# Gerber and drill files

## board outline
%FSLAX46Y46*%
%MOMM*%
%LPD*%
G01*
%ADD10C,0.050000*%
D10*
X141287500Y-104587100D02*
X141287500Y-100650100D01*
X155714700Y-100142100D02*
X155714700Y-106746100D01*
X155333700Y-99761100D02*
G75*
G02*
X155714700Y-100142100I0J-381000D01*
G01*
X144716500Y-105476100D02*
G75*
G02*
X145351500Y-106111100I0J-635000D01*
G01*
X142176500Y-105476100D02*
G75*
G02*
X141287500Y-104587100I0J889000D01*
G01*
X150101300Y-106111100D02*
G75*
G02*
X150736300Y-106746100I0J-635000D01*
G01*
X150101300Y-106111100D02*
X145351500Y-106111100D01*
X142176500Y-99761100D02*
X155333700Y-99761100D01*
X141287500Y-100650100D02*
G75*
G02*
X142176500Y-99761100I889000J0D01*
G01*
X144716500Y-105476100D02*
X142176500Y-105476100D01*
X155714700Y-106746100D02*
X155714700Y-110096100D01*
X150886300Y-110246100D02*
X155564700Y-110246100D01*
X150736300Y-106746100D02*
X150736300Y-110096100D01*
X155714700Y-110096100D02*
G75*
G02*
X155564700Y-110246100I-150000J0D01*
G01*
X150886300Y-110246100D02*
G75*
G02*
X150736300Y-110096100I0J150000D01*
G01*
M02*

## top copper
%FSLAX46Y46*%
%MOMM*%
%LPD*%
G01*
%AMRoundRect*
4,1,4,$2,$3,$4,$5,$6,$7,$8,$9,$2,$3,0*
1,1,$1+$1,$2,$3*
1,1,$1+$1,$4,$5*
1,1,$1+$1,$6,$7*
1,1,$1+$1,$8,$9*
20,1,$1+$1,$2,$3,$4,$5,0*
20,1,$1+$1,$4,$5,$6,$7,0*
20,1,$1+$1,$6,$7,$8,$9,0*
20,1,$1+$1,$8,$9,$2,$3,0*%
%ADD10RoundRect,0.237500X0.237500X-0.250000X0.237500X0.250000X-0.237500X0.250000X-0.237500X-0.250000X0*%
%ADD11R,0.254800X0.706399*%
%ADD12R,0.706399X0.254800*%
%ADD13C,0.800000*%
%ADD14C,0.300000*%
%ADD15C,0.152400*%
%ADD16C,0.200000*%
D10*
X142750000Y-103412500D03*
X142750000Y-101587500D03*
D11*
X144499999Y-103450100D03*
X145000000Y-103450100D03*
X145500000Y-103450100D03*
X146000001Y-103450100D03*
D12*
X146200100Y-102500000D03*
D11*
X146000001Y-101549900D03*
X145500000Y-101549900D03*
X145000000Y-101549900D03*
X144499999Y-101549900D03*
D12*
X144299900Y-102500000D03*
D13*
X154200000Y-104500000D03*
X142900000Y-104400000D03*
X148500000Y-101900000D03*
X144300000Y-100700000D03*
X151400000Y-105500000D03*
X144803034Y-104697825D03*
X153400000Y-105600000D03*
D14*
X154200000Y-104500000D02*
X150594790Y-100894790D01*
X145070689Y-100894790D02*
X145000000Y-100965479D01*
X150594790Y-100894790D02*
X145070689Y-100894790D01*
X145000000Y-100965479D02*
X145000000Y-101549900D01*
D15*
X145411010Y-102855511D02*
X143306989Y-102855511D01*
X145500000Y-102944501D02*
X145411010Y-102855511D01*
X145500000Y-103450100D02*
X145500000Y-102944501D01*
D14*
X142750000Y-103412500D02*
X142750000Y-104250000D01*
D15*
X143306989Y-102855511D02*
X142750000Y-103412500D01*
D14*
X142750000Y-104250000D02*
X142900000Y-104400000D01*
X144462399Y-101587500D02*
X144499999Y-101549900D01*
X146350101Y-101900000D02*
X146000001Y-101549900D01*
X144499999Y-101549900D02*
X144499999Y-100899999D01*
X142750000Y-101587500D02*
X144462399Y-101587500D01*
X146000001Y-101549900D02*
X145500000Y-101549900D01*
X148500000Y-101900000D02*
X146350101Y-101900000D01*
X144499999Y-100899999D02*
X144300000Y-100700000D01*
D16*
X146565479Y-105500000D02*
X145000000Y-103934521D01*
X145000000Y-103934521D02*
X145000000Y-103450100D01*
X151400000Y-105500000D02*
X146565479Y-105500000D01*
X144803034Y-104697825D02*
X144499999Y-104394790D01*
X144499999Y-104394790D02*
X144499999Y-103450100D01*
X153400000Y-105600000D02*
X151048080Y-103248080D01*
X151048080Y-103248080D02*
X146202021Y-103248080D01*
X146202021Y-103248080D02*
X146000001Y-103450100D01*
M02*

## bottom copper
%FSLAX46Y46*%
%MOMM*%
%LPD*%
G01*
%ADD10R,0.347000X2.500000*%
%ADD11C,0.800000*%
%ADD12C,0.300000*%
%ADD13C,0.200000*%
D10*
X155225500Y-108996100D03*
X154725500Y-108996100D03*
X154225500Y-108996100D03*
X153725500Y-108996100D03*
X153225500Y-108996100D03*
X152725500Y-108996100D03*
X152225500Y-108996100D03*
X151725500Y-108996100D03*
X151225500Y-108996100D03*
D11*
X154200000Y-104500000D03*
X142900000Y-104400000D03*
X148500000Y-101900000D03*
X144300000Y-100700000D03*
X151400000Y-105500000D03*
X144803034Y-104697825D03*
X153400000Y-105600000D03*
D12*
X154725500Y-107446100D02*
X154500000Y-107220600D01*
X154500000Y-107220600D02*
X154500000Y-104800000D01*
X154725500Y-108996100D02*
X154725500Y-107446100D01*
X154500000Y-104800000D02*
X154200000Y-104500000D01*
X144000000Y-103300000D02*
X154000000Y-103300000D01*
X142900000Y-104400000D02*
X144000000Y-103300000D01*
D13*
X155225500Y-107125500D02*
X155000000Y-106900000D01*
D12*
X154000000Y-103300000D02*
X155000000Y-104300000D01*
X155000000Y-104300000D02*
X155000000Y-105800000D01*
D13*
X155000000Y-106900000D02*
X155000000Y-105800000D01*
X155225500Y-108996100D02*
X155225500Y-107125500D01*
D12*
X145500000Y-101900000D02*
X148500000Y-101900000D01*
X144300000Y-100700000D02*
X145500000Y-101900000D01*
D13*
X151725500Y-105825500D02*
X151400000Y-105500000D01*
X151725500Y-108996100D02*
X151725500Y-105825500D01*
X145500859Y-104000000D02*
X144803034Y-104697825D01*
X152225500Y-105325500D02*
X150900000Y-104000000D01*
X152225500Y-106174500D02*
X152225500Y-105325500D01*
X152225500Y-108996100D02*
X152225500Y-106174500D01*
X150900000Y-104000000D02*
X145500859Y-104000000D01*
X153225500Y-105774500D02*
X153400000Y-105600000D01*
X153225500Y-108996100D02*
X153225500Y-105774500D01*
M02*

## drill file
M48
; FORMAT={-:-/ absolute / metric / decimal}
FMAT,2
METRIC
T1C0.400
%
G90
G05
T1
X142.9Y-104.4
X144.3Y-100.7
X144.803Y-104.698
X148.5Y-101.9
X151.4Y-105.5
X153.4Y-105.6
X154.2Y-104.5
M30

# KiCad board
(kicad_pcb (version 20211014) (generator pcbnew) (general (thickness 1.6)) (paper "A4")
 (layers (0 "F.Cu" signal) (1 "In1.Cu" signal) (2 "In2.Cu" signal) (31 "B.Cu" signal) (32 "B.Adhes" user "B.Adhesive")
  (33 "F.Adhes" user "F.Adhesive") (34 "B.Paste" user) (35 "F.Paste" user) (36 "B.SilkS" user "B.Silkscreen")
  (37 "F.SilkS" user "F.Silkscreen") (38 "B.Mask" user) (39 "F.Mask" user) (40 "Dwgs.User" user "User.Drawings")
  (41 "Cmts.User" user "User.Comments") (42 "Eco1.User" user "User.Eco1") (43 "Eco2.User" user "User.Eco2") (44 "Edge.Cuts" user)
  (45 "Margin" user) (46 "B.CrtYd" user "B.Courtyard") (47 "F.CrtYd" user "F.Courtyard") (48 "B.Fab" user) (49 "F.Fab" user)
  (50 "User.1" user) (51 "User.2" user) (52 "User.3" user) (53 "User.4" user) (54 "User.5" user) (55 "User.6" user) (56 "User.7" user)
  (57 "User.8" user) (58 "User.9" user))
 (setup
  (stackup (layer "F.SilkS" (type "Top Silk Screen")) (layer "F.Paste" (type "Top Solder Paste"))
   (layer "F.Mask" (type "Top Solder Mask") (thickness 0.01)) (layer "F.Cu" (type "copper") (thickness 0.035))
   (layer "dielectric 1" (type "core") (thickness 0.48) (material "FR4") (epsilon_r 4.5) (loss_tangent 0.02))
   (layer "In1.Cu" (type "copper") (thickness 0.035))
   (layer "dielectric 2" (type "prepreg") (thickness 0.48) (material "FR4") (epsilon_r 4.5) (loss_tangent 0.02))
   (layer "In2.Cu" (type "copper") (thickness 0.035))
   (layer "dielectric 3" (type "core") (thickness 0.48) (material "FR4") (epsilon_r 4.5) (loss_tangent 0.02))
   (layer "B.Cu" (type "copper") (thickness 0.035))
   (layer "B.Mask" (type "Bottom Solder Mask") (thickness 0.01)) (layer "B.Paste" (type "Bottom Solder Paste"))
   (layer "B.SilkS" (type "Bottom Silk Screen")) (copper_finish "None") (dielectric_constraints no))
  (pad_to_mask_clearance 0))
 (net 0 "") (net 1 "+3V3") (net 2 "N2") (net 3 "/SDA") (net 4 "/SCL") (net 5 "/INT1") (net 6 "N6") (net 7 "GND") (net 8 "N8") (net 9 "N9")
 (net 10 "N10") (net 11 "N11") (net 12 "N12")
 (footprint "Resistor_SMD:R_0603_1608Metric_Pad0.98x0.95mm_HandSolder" (layer "F.Cu") (at 142.75 102.5 90)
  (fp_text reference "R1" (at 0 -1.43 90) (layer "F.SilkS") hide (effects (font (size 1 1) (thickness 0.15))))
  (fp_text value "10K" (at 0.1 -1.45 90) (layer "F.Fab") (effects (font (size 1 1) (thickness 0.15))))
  (pad "1" smd roundrect (at -0.9125 0 90) (size 0.975 0.95) (layers "F.Cu" "F.Paste" "F.Mask") (roundrect_rratio 0.25) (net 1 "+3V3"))
  (pad "2" smd roundrect (at 0.9125 0 90) (size 0.975 0.95) (layers "F.Cu" "F.Paste" "F.Mask") (roundrect_rratio 0.25) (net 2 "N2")))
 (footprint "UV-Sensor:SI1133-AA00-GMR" (layer "F.Cu") (at 145.25 102.5 90)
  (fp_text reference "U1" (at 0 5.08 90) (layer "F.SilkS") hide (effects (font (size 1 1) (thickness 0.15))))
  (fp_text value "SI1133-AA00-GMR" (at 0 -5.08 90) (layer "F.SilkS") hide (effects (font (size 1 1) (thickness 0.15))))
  (pad "1" smd rect (at -0.9501 -0.750001 180) (size 0.2548 0.706399) (layers "F.Cu" "F.Paste" "F.Mask") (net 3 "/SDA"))
  (pad "2" smd rect (at -0.9501 -0.25 180) (size 0.2548 0.706399) (layers "F.Cu" "F.Paste" "F.Mask") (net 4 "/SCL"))
  (pad "3" smd rect (at -0.9501 0.25 180) (size 0.2548 0.706399) (layers "F.Cu" "F.Paste" "F.Mask") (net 1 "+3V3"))
  (pad "4" smd rect (at -0.9501 0.750001 180) (size 0.2548 0.706399) (layers "F.Cu" "F.Paste" "F.Mask") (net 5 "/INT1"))
  (pad "5" smd rect (at 0 0.9501 90) (size 0.2548 0.706399) (layers "F.Cu" "F.Paste" "F.Mask") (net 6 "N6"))
  (pad "6" smd rect (at 0.9501 0.750001 180) (size 0.2548 0.706399) (layers "F.Cu" "F.Paste" "F.Mask") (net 2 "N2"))
  (pad "7" smd rect (at 0.9501 0.25 180) (size 0.2548 0.706399) (layers "F.Cu" "F.Paste" "F.Mask") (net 2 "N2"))
  (pad "8" smd rect (at 0.9501 -0.25 180) (size 0.2548 0.706399) (layers "F.Cu" "F.Paste" "F.Mask") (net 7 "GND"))
  (pad "9" smd rect (at 0.9501 -0.750001 180) (size 0.2548 0.706399) (layers "F.Cu" "F.Paste" "F.Mask") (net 2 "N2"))
  (pad "10" smd rect (at 0 -0.9501 90) (size 0.2548 0.706399) (layers "F.Cu" "F.Paste" "F.Mask") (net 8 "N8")))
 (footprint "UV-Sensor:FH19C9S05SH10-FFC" (layer "F.Cu") (at 153.2255 106.7461)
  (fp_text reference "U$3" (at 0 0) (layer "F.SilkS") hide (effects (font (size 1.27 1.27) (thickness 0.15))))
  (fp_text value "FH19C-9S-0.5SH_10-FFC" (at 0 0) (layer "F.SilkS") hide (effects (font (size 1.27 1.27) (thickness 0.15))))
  (fp_line (start 2.4892 0) (end 2.4892 3.35) (layer "Edge.Cuts") (width 0.05))
  (fp_line (start -2.3392 3.5) (end 2.3392 3.5) (layer "Edge.Cuts") (width 0.05))
  (fp_line (start -2.4892 0) (end -2.4892 3.35) (layer "Edge.Cuts") (width 0.05))
  (fp_arc (start 2.4892 3.35) (mid 2.445266 3.456066) (end 2.3392 3.5) (layer "Edge.Cuts") (width 0.05))
  (fp_arc (start -2.3392 3.5) (mid -2.445266 3.456066) (end -2.4892 3.35) (layer "Edge.Cuts") (width 0.05))
  (pad "1" smd rect (at 2 2.25 90) (size 2.5 0.347) (layers "B.Cu" "B.Paste" "B.Mask") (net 1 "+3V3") (solder_mask_margin 0.0635))
  (pad "2" smd rect (at 1.5 2.25 90) (size 2.5 0.347) (layers "B.Cu" "B.Paste" "B.Mask") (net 7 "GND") (solder_mask_margin 0.0635))
  (pad "3" smd rect (at 1 2.25 90) (size 2.5 0.347) (layers "B.Cu" "B.Paste" "B.Mask") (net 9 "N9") (solder_mask_margin 0.0635))
  (pad "4" smd rect (at 0.5 2.25 90) (size 2.5 0.347) (layers "B.Cu" "B.Paste" "B.Mask") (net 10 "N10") (solder_mask_margin 0.0635))
  (pad "5" smd rect (at 0 2.25 90) (size 2.5 0.347) (layers "B.Cu" "B.Paste" "B.Mask") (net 5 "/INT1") (solder_mask_margin 0.0635))
  (pad "6" smd rect (at -0.5 2.25 90) (size 2.5 0.347) (layers "B.Cu" "B.Paste" "B.Mask") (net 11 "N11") (solder_mask_margin 0.0635))
  (pad "7" smd rect (at -1 2.25 90) (size 2.5 0.347) (layers "B.Cu" "B.Paste" "B.Mask") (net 3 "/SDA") (solder_mask_margin 0.0635))
  (pad "8" smd rect (at -1.5 2.25 90) (size 2.5 0.347) (layers "B.Cu" "B.Paste" "B.Mask") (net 4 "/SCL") (solder_mask_margin 0.0635))
  (pad "9" smd rect (at -2 2.25 90) (size 2.5 0.347) (layers "B.Cu" "B.Paste" "B.Mask") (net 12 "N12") (solder_mask_margin 0.0635)))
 (gr_line (start 141.2875 104.5871) (end 141.2875 100.6501) (layer "Edge.Cuts") (width 0.05))
 (gr_line (start 155.7147 100.1421) (end 155.7147 106.7461) (layer "Edge.Cuts") (width 0.05))
 (gr_arc (start 155.3337 99.7611) (mid 155.603108 99.872692) (end 155.7147 100.1421) (layer "Edge.Cuts") (width 0.05))
 (gr_arc (start 144.7165 105.4761) (mid 145.165513 105.662087) (end 145.3515 106.1111) (layer "Edge.Cuts") (width 0.05))
 (gr_arc (start 142.1765 105.4761) (mid 141.547882 105.215718) (end 141.2875 104.5871) (layer "Edge.Cuts") (width 0.05))
 (gr_arc (start 150.1013 106.1111) (mid 150.550313 106.297087) (end 150.7363 106.7461) (layer "Edge.Cuts") (width 0.05))
 (gr_line (start 150.1013 106.1111) (end 145.3515 106.1111) (layer "Edge.Cuts") (width 0.05))
 (gr_line (start 142.1765 99.7611) (end 155.3337 99.7611) (layer "Edge.Cuts") (width 0.05))
 (gr_arc (start 141.2875 100.6501) (mid 141.547882 100.021482) (end 142.1765 99.7611) (layer "Edge.Cuts") (width 0.05))
 (gr_line (start 144.7165 105.4761) (end 142.1765 105.4761) (layer "Edge.Cuts") (width 0.05))
 (segment (start 154.2 104.5) (end 150.59479 100.89479) (width 0.3) (layer "F.Cu") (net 7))
 (segment (start 145.070689 100.89479) (end 145 100.965479) (width 0.3) (layer "F.Cu") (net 7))
 (segment (start 150.59479 100.89479) (end 145.070689 100.89479) (width 0.3) (layer "F.Cu") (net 7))
 (segment (start 145 100.965479) (end 145 101.5499) (width 0.3) (layer "F.Cu") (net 7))
 (via (at 154.2 104.5) (size 0.8) (drill 0.4) (layers "F.Cu" "B.Cu") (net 7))
 (segment (start 154.7255 107.4461) (end 154.5 107.2206) (width 0.3) (layer "B.Cu") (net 7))
 (segment (start 154.5 107.2206) (end 154.5 104.8) (width 0.3) (layer "B.Cu") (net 7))
 (segment (start 154.7255 108.9961) (end 154.7255 107.4461) (width 0.3) (layer "B.Cu") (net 7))
 (segment (start 154.5 104.8) (end 154.2 104.5) (width 0.3) (layer "B.Cu") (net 7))
 (segment (start 145.41101 102.855511) (end 143.306989 102.855511) (width 0.1524) (layer "F.Cu") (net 1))
 (segment (start 145.5 102.944501) (end 145.41101 102.855511) (width 0.1524) (layer "F.Cu") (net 1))
 (segment (start 145.5 103.4501) (end 145.5 102.944501) (width 0.1524) (layer "F.Cu") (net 1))
 (segment (start 142.75 103.4125) (end 142.75 104.25) (width 0.3) (layer "F.Cu") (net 1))
 (segment (start 143.306989 102.855511) (end 142.75 103.4125) (width 0.1524) (layer "F.Cu") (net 1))
 (segment (start 142.75 104.25) (end 142.9 104.4) (width 0.3) (layer "F.Cu") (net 1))
 (via (at 142.9 104.4) (size 0.8) (drill 0.4) (layers "F.Cu" "B.Cu") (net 1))
 (segment (start 144 103.3) (end 154 103.3) (width 0.3) (layer "B.Cu") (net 1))
 (segment (start 142.9 104.4) (end 144 103.3) (width 0.3) (layer "B.Cu") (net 1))
 (segment (start 155.2255 107.1255) (end 155 106.9) (width 0.2) (layer "B.Cu") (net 1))
 (segment (start 154 103.3) (end 155 104.3) (width 0.3) (layer "B.Cu") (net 1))
 (segment (start 155 104.3) (end 155 105.8) (width 0.3) (layer "B.Cu") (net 1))
 (segment (start 155 106.9) (end 155 105.8) (width 0.2) (layer "B.Cu") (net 1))
 (segment (start 155.2255 108.9961) (end 155.2255 107.1255) (width 0.2) (layer "B.Cu") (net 1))
 (segment (start 144.462399 101.5875) (end 144.499999 101.5499) (width 0.3) (layer "F.Cu") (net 2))
 (segment (start 146.350101 101.9) (end 146.000001 101.5499) (width 0.3) (layer "F.Cu") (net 2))
 (segment (start 144.499999 101.5499) (end 144.499999 100.899999) (width 0.3) (layer "F.Cu") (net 2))
 (segment (start 142.75 101.5875) (end 144.462399 101.5875) (width 0.3) (layer "F.Cu") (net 2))
 (segment (start 146.000001 101.5499) (end 145.5 101.5499) (width 0.3) (layer "F.Cu") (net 2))
 (segment (start 148.5 101.9) (end 146.350101 101.9) (width 0.3) (layer "F.Cu") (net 2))
 (segment (start 144.499999 100.899999) (end 144.3 100.7) (width 0.3) (layer "F.Cu") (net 2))
 (via (at 148.5 101.9) (size 0.8) (drill 0.4) (layers "F.Cu" "B.Cu") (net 2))
 (via (at 144.3 100.7) (size 0.8) (drill 0.4) (layers "F.Cu" "B.Cu") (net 2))
 (segment (start 145.5 101.9) (end 148.5 101.9) (width 0.3) (layer "B.Cu") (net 2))
 (segment (start 144.3 100.7) (end 145.5 101.9) (width 0.3) (layer "B.Cu") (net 2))
 (segment (start 146.565479 105.5) (end 145 103.934521) (width 0.2) (layer "F.Cu") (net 4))
 (segment (start 145 103.934521) (end 145 103.4501) (width 0.2) (layer "F.Cu") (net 4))
 (segment (start 151.4 105.5) (end 146.565479 105.5) (width 0.2) (layer "F.Cu") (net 4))
 (via (at 151.4 105.5) (size 0.8) (drill 0.4) (layers "F.Cu" "B.Cu") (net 4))
 (segment (start 151.7255 105.8255) (end 151.4 105.5) (width 0.2) (layer "B.Cu") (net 4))
 (segment (start 151.7255 108.9961) (end 151.7255 105.8255) (width 0.2) (layer "B.Cu") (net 4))
 (segment (start 144.803034 104.697825) (end 144.499999 104.39479) (width 0.2) (layer "F.Cu") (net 3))
 (segment (start 144.499999 104.39479) (end 144.499999 103.4501) (width 0.2) (layer "F.Cu") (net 3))
 (via (at 144.803034 104.697825) (size 0.8) (drill 0.4) (layers "F.Cu" "B.Cu") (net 3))
 (segment (start 145.500859 104) (end 144.803034 104.697825) (width 0.2) (layer "B.Cu") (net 3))
 (segment (start 152.2255 105.3255) (end 150.9 104) (width 0.2) (layer "B.Cu") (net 3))
 (segment (start 152.2255 106.1745) (end 152.2255 105.3255) (width 0.2) (layer "B.Cu") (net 3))
 (segment (start 152.2255 108.9961) (end 152.2255 106.1745) (width 0.2) (layer "B.Cu") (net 3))
 (segment (start 150.9 104) (end 145.500859 104) (width 0.2) (layer "B.Cu") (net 3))
 (segment (start 153.4 105.6) (end 151.04808 103.24808) (width 0.2) (layer "F.Cu") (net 5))
 (segment (start 151.04808 103.24808) (end 146.202021 103.24808) (width 0.2) (layer "F.Cu") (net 5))
 (segment (start 146.202021 103.24808) (end 146.000001 103.4501) (width 0.2) (layer "F.Cu") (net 5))
 (via (at 153.4 105.6) (size 0.8) (drill 0.4) (layers "F.Cu" "B.Cu") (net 5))
 (segment (start 153.2255 105.7745) (end 153.4 105.6) (width 0.2) (layer "B.Cu") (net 5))
 (segment (start 153.2255 108.9961) (end 153.2255 105.7745) (width 0.2) (layer "B.Cu") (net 5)))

